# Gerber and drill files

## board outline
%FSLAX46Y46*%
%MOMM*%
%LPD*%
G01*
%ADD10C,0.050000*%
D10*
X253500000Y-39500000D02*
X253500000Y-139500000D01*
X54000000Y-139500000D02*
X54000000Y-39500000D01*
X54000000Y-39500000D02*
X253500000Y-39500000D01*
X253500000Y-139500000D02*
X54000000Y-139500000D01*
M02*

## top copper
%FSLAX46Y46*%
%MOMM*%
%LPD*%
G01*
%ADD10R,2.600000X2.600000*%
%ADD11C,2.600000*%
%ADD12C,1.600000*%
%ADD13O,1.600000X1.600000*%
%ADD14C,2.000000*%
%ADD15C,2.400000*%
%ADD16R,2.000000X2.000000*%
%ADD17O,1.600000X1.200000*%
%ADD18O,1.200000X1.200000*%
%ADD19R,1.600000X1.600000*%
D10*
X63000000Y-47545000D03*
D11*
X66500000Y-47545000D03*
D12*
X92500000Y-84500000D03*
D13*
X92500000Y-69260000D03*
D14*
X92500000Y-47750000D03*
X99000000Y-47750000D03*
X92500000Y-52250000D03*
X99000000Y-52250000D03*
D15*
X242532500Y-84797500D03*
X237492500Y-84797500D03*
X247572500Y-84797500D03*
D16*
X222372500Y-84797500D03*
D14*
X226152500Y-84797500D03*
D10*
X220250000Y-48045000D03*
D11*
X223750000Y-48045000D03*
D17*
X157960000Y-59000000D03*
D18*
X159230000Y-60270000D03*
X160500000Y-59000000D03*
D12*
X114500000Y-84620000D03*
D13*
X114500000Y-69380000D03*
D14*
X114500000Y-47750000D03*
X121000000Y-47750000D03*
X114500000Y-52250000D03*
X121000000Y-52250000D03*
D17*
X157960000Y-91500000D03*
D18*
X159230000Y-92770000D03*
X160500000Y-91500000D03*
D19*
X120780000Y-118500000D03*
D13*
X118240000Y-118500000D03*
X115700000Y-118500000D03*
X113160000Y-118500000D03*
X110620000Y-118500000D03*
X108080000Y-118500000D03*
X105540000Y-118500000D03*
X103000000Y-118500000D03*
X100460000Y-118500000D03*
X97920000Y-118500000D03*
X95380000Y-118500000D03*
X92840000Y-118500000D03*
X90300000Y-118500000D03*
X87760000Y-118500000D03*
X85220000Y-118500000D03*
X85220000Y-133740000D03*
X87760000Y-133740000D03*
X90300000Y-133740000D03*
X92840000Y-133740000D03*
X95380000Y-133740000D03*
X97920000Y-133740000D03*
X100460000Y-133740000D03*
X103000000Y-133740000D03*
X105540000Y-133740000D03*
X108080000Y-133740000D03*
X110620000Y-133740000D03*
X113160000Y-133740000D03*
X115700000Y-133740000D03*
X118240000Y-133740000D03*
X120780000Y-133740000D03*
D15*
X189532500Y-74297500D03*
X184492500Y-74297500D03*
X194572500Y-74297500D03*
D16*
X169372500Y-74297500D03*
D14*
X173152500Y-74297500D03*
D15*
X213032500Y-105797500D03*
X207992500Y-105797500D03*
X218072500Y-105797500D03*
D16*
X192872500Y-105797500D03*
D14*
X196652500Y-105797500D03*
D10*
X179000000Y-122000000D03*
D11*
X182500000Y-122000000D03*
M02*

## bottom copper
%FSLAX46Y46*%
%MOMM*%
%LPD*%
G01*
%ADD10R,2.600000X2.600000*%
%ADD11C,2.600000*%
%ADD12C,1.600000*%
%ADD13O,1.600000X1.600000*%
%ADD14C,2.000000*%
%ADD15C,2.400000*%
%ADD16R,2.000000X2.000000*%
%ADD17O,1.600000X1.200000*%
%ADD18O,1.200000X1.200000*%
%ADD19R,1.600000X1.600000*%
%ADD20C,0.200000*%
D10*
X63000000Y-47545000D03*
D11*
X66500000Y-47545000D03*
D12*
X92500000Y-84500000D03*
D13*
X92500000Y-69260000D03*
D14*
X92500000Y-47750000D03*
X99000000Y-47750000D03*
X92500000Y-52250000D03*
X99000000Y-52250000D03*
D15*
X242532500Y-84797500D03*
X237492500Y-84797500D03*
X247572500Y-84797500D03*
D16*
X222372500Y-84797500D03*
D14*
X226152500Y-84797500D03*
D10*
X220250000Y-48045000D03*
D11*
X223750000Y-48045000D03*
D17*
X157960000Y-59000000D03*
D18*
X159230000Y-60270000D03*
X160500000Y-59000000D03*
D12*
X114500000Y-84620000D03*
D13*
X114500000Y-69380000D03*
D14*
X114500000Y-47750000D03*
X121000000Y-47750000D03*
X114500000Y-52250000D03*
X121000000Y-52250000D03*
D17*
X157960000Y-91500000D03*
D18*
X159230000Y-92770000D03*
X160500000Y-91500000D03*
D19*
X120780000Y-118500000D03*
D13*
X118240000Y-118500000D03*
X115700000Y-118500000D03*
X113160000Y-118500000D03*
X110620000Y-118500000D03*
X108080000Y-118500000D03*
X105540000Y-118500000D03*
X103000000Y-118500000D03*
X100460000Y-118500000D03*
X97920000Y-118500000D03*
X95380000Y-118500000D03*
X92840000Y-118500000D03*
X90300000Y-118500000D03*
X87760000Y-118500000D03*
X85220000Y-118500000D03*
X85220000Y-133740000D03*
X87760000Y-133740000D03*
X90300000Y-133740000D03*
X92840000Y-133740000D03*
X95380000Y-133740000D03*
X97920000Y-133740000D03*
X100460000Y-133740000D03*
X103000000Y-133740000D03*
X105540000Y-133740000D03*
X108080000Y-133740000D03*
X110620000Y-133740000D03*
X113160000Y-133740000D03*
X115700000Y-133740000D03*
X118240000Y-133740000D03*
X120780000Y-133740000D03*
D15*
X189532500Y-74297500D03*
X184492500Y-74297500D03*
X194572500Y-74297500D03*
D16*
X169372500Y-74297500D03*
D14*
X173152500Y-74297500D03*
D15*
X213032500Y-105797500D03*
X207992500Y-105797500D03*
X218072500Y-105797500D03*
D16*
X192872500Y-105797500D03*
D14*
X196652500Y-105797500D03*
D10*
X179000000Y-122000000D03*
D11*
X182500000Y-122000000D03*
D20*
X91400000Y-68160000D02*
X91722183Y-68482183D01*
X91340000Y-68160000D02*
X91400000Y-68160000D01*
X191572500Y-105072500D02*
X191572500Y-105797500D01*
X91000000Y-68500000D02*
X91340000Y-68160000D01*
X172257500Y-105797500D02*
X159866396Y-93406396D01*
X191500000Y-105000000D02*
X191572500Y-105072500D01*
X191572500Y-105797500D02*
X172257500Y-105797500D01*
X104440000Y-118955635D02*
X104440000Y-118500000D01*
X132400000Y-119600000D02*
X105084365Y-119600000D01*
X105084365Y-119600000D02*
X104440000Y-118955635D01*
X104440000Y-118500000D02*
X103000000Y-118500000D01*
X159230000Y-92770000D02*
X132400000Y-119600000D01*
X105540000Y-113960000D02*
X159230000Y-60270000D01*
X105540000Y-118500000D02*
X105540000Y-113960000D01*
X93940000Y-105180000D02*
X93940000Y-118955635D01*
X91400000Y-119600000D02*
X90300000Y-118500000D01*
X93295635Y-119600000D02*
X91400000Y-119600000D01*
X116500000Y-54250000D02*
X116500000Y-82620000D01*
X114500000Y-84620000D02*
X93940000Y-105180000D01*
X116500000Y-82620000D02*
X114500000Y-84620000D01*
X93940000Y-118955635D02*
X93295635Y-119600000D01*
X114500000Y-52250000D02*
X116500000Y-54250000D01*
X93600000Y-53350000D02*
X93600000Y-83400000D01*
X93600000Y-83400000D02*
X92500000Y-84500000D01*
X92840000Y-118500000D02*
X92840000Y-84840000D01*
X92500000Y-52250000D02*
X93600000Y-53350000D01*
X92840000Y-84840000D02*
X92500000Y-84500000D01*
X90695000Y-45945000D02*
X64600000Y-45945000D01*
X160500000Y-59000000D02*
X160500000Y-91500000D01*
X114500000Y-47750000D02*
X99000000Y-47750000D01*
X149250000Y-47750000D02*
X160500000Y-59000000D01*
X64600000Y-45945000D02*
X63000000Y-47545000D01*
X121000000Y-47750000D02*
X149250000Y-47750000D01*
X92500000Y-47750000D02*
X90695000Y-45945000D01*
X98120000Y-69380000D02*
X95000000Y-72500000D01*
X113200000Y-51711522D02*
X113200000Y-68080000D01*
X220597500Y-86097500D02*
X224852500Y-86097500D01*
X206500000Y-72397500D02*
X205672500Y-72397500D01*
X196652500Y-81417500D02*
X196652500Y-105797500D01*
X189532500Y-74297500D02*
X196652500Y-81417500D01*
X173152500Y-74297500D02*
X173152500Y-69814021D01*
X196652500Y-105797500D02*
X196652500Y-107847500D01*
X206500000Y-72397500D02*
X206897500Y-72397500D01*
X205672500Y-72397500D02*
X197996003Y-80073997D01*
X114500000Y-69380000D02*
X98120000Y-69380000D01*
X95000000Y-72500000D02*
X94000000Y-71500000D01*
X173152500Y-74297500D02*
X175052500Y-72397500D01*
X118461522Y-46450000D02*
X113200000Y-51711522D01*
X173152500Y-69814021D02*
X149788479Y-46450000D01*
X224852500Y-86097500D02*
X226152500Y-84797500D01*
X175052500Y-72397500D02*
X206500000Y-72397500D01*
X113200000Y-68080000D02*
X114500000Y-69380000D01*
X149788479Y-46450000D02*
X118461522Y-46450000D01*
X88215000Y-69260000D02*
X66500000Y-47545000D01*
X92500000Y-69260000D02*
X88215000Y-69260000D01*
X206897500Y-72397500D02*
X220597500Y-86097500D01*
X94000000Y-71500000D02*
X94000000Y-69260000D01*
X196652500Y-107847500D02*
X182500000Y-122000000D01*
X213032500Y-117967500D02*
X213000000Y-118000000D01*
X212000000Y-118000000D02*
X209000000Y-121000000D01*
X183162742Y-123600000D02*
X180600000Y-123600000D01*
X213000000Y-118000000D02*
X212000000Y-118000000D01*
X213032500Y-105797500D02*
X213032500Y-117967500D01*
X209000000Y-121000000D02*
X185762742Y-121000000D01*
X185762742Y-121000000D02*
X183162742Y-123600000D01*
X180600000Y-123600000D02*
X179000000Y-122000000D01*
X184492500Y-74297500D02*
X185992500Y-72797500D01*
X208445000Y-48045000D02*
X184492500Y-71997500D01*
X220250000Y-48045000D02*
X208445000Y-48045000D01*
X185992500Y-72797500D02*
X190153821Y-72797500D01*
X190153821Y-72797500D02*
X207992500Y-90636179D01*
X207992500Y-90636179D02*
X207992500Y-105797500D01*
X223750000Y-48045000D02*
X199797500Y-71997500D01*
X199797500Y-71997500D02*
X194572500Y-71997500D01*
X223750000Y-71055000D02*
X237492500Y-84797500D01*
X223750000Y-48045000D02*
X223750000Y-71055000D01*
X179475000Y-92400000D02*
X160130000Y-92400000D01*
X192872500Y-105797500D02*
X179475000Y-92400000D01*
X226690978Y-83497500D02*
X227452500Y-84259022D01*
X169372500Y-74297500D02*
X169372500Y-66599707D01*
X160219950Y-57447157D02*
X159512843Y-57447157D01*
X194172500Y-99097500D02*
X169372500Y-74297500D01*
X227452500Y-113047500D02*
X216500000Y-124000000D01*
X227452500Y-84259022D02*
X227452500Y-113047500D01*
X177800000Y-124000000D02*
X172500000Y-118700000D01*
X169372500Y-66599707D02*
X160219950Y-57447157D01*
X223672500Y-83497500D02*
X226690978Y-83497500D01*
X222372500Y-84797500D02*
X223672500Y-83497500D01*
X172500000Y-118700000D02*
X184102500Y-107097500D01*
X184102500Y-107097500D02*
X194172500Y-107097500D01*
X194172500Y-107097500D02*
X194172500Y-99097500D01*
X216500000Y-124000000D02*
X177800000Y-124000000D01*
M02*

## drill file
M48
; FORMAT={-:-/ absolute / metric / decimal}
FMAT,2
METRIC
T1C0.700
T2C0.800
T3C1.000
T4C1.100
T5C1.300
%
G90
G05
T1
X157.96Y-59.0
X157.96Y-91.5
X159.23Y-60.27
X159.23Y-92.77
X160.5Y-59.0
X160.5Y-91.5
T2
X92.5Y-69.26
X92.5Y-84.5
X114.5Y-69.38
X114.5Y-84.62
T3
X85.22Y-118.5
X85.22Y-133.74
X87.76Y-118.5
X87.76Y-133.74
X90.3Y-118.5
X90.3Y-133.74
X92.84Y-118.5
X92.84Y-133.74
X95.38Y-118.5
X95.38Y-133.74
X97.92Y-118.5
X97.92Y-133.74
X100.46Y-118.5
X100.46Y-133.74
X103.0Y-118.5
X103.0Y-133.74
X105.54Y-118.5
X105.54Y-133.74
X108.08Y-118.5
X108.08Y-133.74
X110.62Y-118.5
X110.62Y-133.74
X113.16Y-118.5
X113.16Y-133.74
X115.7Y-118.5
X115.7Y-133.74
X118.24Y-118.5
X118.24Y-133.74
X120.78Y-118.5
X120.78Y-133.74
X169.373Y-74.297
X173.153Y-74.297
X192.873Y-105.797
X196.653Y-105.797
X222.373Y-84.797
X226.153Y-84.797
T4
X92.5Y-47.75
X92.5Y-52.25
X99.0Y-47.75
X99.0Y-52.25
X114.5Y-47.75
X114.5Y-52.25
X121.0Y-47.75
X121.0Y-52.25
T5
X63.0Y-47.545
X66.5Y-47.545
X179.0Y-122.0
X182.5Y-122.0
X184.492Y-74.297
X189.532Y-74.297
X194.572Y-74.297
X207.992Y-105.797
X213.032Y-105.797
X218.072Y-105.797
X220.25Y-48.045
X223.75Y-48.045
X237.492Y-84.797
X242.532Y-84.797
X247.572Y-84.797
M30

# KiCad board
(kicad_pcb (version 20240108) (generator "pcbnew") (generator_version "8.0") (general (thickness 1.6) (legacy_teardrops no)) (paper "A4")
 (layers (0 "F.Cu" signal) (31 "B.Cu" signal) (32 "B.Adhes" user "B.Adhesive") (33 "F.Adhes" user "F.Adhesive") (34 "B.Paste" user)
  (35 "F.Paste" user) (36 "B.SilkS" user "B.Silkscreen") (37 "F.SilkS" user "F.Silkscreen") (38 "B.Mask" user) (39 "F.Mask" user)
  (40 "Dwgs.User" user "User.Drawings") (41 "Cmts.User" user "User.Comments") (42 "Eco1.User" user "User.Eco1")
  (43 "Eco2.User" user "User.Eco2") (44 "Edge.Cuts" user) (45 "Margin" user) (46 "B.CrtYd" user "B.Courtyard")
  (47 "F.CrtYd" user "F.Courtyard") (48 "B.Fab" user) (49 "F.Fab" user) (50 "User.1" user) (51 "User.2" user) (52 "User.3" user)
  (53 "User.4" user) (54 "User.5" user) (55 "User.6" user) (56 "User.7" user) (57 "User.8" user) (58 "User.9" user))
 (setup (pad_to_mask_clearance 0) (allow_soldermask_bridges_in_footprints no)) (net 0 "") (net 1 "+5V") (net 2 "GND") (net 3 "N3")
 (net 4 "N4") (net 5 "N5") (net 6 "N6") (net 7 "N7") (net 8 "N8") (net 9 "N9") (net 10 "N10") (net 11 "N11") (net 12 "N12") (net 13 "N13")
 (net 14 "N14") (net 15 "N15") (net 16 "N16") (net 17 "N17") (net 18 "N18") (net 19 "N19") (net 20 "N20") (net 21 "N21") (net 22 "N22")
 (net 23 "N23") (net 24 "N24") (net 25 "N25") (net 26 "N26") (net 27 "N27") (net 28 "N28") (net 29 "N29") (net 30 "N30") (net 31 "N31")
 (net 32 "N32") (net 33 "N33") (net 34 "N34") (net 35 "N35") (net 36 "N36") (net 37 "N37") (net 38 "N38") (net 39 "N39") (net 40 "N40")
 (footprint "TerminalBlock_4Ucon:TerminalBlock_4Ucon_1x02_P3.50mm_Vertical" (layer "F.Cu") (at 63 47.545)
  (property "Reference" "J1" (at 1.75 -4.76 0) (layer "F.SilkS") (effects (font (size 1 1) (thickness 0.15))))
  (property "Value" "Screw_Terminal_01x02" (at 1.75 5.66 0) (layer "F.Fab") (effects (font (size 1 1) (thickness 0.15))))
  (pad "1" thru_hole rect (at 0 0) (size 2.6 2.6) (drill 1.3) (layers "*.Cu" "*.Mask") (remove_unused_layers no) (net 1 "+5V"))
  (pad "2" thru_hole circle (at 3.5 0) (size 2.6 2.6) (drill 1.3) (layers "*.Cu" "*.Mask") (remove_unused_layers no) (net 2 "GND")))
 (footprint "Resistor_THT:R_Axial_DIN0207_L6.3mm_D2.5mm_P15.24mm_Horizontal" (layer "F.Cu") (at 92.5 84.5 90)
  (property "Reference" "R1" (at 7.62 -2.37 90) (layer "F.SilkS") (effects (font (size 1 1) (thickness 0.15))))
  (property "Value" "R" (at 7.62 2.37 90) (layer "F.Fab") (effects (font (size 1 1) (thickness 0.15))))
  (pad "1" thru_hole circle (at 0 0 90) (size 1.6 1.6) (drill 0.8) (layers "*.Cu" "*.Mask") (remove_unused_layers no) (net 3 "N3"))
  (pad "2" thru_hole oval (at 15.24 0 90) (size 1.6 1.6) (drill 0.8) (layers "*.Cu" "*.Mask") (remove_unused_layers no) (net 2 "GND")))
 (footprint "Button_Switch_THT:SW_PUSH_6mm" (layer "F.Cu") (at 92.5 47.75)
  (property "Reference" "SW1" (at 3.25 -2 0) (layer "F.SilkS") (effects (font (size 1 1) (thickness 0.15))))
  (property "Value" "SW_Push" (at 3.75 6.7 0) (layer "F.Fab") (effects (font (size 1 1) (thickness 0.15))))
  (pad "1" thru_hole circle (at 0 0 90) (size 2 2) (drill 1.1) (layers "*.Cu" "*.Mask") (remove_unused_layers no) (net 1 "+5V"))
  (pad "1" thru_hole circle (at 6.5 0 90) (size 2 2) (drill 1.1) (layers "*.Cu" "*.Mask") (remove_unused_layers no) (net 1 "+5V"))
  (pad "2" thru_hole circle (at 0 4.5 90) (size 2 2) (drill 1.1) (layers "*.Cu" "*.Mask") (remove_unused_layers no) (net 3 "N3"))
  (pad "2" thru_hole circle (at 6.5 4.5 90) (size 2 2) (drill 1.1) (layers "*.Cu" "*.Mask") (remove_unused_layers no) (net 3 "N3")))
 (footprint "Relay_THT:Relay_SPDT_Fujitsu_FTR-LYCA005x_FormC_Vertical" (layer "F.Cu") (at 222.3725 84.7975)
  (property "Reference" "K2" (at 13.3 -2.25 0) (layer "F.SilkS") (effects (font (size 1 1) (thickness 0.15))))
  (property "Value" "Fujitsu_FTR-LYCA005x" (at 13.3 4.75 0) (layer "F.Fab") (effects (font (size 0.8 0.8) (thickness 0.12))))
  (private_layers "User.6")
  (pad "11" thru_hole circle (at 20.16 0) (size 2.4 2.4) (drill 1.3) (layers "*.Cu" "*.Mask") (remove_unused_layers no) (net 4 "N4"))
  (pad "12" thru_hole circle (at 15.12 0) (size 2.4 2.4) (drill 1.3) (layers "*.Cu" "*.Mask") (remove_unused_layers no) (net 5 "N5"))
  (pad "14" thru_hole circle (at 25.2 0) (size 2.4 2.4) (drill 1.3) (layers "*.Cu" "*.Mask") (remove_unused_layers no) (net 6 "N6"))
  (pad "A1" thru_hole rect (at 0 0) (size 2 2) (drill 1) (layers "*.Cu" "*.Mask") (remove_unused_layers no) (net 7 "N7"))
  (pad "A2" thru_hole circle (at 3.78 0) (size 2 2) (drill 1) (layers "*.Cu" "*.Mask") (remove_unused_layers no) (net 2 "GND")))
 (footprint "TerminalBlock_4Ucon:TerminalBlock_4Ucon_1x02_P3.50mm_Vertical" (layer "F.Cu") (at 220.25 48.045)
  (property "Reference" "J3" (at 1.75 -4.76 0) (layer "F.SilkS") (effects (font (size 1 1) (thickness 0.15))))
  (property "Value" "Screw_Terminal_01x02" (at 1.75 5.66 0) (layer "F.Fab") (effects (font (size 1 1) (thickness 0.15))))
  (pad "1" thru_hole rect (at 0 0) (size 2.6 2.6) (drill 1.3) (layers "*.Cu" "*.Mask") (remove_unused_layers no) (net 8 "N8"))
  (pad "2" thru_hole circle (at 3.5 0) (size 2.6 2.6) (drill 1.3) (layers "*.Cu" "*.Mask") (remove_unused_layers no) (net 5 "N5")))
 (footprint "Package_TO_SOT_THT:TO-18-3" (layer "F.Cu") (at 157.96 59)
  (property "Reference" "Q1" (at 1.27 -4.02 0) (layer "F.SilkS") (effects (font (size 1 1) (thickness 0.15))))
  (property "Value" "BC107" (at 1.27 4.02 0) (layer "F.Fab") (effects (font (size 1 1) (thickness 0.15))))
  (pad "1" thru_hole oval (at 0 0) (size 1.6 1.2) (drill 0.7) (layers "*.Cu" "*.Mask") (remove_unused_layers no) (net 7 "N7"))
  (pad "2" thru_hole oval (at 1.27 1.27) (size 1.2 1.2) (drill 0.7) (layers "*.Cu" "*.Mask") (remove_unused_layers no) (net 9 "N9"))
  (pad "3" thru_hole oval (at 2.54 0) (size 1.2 1.2) (drill 0.7) (layers "*.Cu" "*.Mask") (remove_unused_layers no) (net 1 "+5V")))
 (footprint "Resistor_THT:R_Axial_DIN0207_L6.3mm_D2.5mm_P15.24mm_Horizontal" (layer "F.Cu") (at 114.5 84.62 90)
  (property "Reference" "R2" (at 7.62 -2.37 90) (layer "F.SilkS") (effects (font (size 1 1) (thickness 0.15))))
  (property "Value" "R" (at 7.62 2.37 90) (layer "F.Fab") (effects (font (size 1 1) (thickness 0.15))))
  (pad "1" thru_hole circle (at 0 0 90) (size 1.6 1.6) (drill 0.8) (layers "*.Cu" "*.Mask") (remove_unused_layers no) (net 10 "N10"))
  (pad "2" thru_hole oval (at 15.24 0 90) (size 1.6 1.6) (drill 0.8) (layers "*.Cu" "*.Mask") (remove_unused_layers no) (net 2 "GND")))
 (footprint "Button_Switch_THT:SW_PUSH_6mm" (layer "F.Cu") (at 114.5 47.75)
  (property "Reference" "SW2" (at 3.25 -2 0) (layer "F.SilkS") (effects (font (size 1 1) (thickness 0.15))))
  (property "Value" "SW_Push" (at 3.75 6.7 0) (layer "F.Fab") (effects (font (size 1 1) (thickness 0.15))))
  (pad "1" thru_hole circle (at 0 0 90) (size 2 2) (drill 1.1) (layers "*.Cu" "*.Mask") (remove_unused_layers no) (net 1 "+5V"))
  (pad "1" thru_hole circle (at 6.5 0 90) (size 2 2) (drill 1.1) (layers "*.Cu" "*.Mask") (remove_unused_layers no) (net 1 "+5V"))
  (pad "2" thru_hole circle (at 0 4.5 90) (size 2 2) (drill 1.1) (layers "*.Cu" "*.Mask") (remove_unused_layers no) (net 10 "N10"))
  (pad "2" thru_hole circle (at 6.5 4.5 90) (size 2 2) (drill 1.1) (layers "*.Cu" "*.Mask") (remove_unused_layers no) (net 10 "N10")))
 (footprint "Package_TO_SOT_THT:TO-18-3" (layer "F.Cu") (at 157.96 91.5)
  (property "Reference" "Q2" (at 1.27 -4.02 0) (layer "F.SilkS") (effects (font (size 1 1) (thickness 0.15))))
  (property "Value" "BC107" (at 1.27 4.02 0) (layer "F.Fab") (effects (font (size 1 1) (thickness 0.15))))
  (pad "1" thru_hole oval (at 0 0) (size 1.6 1.2) (drill 0.7) (layers "*.Cu" "*.Mask") (remove_unused_layers no) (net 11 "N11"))
  (pad "2" thru_hole oval (at 1.27 1.27) (size 1.2 1.2) (drill 0.7) (layers "*.Cu" "*.Mask") (remove_unused_layers no) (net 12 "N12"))
  (pad "3" thru_hole oval (at 2.54 0) (size 1.2 1.2) (drill 0.7) (layers "*.Cu" "*.Mask") (remove_unused_layers no) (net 1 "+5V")))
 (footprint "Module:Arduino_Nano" (layer "F.Cu") (at 120.78 118.5 -90)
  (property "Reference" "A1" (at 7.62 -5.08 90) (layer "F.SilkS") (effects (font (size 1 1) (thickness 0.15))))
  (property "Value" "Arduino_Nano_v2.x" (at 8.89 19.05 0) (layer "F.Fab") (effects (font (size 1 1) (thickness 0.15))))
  (pad "1" thru_hole rect (at 0 0 270) (size 1.6 1.6) (drill 1) (layers "*.Cu" "*.Mask") (remove_unused_layers no) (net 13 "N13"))
  (pad "2" thru_hole oval (at 0 2.54 270) (size 1.6 1.6) (drill 1) (layers "*.Cu" "*.Mask") (remove_unused_layers no) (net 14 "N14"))
  (pad "3" thru_hole oval (at 0 5.08 270) (size 1.6 1.6) (drill 1) (layers "*.Cu" "*.Mask") (remove_unused_layers no) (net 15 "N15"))
  (pad "4" thru_hole oval (at 0 7.62 270) (size 1.6 1.6) (drill 1) (layers "*.Cu" "*.Mask") (remove_unused_layers no) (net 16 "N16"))
  (pad "5" thru_hole oval (at 0 10.16 270) (size 1.6 1.6) (drill 1) (layers "*.Cu" "*.Mask") (remove_unused_layers no) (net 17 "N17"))
  (pad "6" thru_hole oval (at 0 12.7 270) (size 1.6 1.6) (drill 1) (layers "*.Cu" "*.Mask") (remove_unused_layers no) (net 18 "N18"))
  (pad "7" thru_hole oval (at 0 15.24 270) (size 1.6 1.6) (drill 1) (layers "*.Cu" "*.Mask") (remove_unused_layers no) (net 9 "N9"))
  (pad "8" thru_hole oval (at 0 17.78 270) (size 1.6 1.6) (drill 1) (layers "*.Cu" "*.Mask") (remove_unused_layers no) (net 12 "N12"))
  (pad "9" thru_hole oval (at 0 20.32 270) (size 1.6 1.6) (drill 1) (layers "*.Cu" "*.Mask") (remove_unused_layers no) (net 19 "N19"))
  (pad "10" thru_hole oval (at 0 22.86 270) (size 1.6 1.6) (drill 1) (layers "*.Cu" "*.Mask") (remove_unused_layers no) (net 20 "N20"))
  (pad "11" thru_hole oval (at 0 25.4 270) (size 1.6 1.6) (drill 1) (layers "*.Cu" "*.Mask") (remove_unused_layers no) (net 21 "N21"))
  (pad "12" thru_hole oval (at 0 27.94 270) (size 1.6 1.6) (drill 1) (layers "*.Cu" "*.Mask") (remove_unused_layers no) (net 3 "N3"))
  (pad "13" thru_hole oval (at 0 30.48 270) (size 1.6 1.6) (drill 1) (layers "*.Cu" "*.Mask") (remove_unused_layers no) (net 10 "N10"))
  (pad "14" thru_hole oval (at 0 33.02 270) (size 1.6 1.6) (drill 1) (layers "*.Cu" "*.Mask") (remove_unused_layers no) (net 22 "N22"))
  (pad "15" thru_hole oval (at 0 35.56 270) (size 1.6 1.6) (drill 1) (layers "*.Cu" "*.Mask") (remove_unused_layers no) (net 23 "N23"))
  (pad "16" thru_hole oval (at 15.24 35.56 270) (size 1.6 1.6) (drill 1) (layers "*.Cu" "*.Mask") (remove_unused_layers no) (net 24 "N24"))
  (pad "17" thru_hole oval (at 15.24 33.02 270) (size 1.6 1.6) (drill 1) (layers "*.Cu" "*.Mask") (remove_unused_layers no) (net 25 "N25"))
  (pad "18" thru_hole oval (at 15.24 30.48 270) (size 1.6 1.6) (drill 1) (layers "*.Cu" "*.Mask") (remove_unused_layers no) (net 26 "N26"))
  (pad "19" thru_hole oval (at 15.24 27.94 270) (size 1.6 1.6) (drill 1) (layers "*.Cu" "*.Mask") (remove_unused_layers no) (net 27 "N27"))
  (pad "20" thru_hole oval (at 15.24 25.4 270) (size 1.6 1.6) (drill 1) (layers "*.Cu" "*.Mask") (remove_unused_layers no) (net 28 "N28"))
  (pad "21" thru_hole oval (at 15.24 22.86 270) (size 1.6 1.6) (drill 1) (layers "*.Cu" "*.Mask") (remove_unused_layers no) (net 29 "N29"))
  (pad "22" thru_hole oval (at 15.24 20.32 270) (size 1.6 1.6) (drill 1) (layers "*.Cu" "*.Mask") (remove_unused_layers no) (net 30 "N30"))
  (pad "23" thru_hole oval (at 15.24 17.78 270) (size 1.6 1.6) (drill 1) (layers "*.Cu" "*.Mask") (remove_unused_layers no) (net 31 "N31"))
  (pad "24" thru_hole oval (at 15.24 15.24 270) (size 1.6 1.6) (drill 1) (layers "*.Cu" "*.Mask") (remove_unused_layers no) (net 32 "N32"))
  (pad "25" thru_hole oval (at 15.24 12.7 270) (size 1.6 1.6) (drill 1) (layers "*.Cu" "*.Mask") (remove_unused_layers no) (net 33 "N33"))
  (pad "26" thru_hole oval (at 15.24 10.16 270) (size 1.6 1.6) (drill 1) (layers "*.Cu" "*.Mask") (remove_unused_layers no) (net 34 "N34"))
  (pad "27" thru_hole oval (at 15.24 7.62 270) (size 1.6 1.6) (drill 1) (layers "*.Cu" "*.Mask") (remove_unused_layers no) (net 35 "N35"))
  (pad "28" thru_hole oval (at 15.24 5.08 270) (size 1.6 1.6) (drill 1) (layers "*.Cu" "*.Mask") (remove_unused_layers no) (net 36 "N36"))
  (pad "29" thru_hole oval (at 15.24 2.54 270) (size 1.6 1.6) (drill 1) (layers "*.Cu" "*.Mask") (remove_unused_layers no) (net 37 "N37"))
  (pad "30" thru_hole oval (at 15.24 0 270) (size 1.6 1.6) (drill 1) (layers "*.Cu" "*.Mask") (remove_unused_layers no) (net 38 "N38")))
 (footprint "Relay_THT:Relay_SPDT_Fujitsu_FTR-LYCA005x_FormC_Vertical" (layer "F.Cu") (at 169.3725 74.2975)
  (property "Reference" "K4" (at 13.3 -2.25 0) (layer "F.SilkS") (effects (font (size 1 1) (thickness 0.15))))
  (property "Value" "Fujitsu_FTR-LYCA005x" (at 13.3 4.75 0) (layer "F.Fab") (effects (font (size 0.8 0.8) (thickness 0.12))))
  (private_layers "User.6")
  (pad "11" thru_hole circle (at 20.16 0) (size 2.4 2.4) (drill 1.3) (layers "*.Cu" "*.Mask") (remove_unused_layers no) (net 2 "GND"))
  (pad "12" thru_hole circle (at 15.12 0) (size 2.4 2.4) (drill 1.3) (layers "*.Cu" "*.Mask") (remove_unused_layers no) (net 8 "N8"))
  (pad "14" thru_hole circle (at 25.2 0) (size 2.4 2.4) (drill 1.3) (layers "*.Cu" "*.Mask") (remove_unused_layers no) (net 5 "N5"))
  (pad "A1" thru_hole rect (at 0 0) (size 2 2) (drill 1) (layers "*.Cu" "*.Mask") (remove_unused_layers no) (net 7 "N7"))
  (pad "A2" thru_hole circle (at 3.78 0) (size 2 2) (drill 1) (layers "*.Cu" "*.Mask") (remove_unused_layers no) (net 2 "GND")))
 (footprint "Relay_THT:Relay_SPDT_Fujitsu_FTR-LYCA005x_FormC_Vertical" (layer "F.Cu") (at 192.8725 105.7975)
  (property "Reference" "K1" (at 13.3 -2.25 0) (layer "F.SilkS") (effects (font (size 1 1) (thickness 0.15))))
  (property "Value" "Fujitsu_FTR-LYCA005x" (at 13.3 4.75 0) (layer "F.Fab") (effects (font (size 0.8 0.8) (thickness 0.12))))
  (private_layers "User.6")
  (pad "11" thru_hole circle (at 20.16 0) (size 2.4 2.4) (drill 1.3) (layers "*.Cu" "*.Mask") (remove_unused_layers no) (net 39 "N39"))
  (pad "12" thru_hole circle (at 15.12 0) (size 2.4 2.4) (drill 1.3) (layers "*.Cu" "*.Mask") (remove_unused_layers no) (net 8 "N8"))
  (pad "14" thru_hole circle (at 25.2 0) (size 2.4 2.4) (drill 1.3) (layers "*.Cu" "*.Mask") (remove_unused_layers no) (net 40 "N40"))
  (pad "A1" thru_hole rect (at 0 0) (size 2 2) (drill 1) (layers "*.Cu" "*.Mask") (remove_unused_layers no) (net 11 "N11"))
  (pad "A2" thru_hole circle (at 3.78 0) (size 2 2) (drill 1) (layers "*.Cu" "*.Mask") (remove_unused_layers no) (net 2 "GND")))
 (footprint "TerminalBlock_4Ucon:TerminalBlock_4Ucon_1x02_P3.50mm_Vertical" (layer "F.Cu") (at 179 122)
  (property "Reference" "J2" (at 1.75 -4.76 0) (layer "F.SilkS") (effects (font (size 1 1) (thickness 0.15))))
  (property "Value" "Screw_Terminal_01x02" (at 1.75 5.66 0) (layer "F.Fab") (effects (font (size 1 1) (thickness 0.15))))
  (pad "1" thru_hole rect (at 0 0) (size 2.6 2.6) (drill 1.3) (layers "*.Cu" "*.Mask") (remove_unused_layers no) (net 39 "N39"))
  (pad "2" thru_hole circle (at 3.5 0) (size 2.6 2.6) (drill 1.3) (layers "*.Cu" "*.Mask") (remove_unused_layers no) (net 2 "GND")))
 (gr_line (start 253.5 39.5) (end 253.5 139.5) (stroke (width 0.05) (type default)) (layer "Edge.Cuts"))
 (gr_line (start 54 139.5) (end 54 39.5) (stroke (width 0.05) (type default)) (layer "Edge.Cuts"))
 (gr_line (start 54 39.5) (end 253.5 39.5) (stroke (width 0.05) (type default)) (layer "Edge.Cuts"))
 (gr_line (start 253.5 139.5) (end 54 139.5) (stroke (width 0.05) (type default)) (layer "Edge.Cuts"))
 (segment (start 91.4 68.16) (end 91.722183 68.482183) (width 0.2) (layer "B.Cu") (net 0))
 (segment (start 91.34 68.16) (end 91.4 68.16) (width 0.2) (layer "B.Cu") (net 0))
 (segment (start 191.5725 105.0725) (end 191.5725 105.7975) (width 0.2) (layer "B.Cu") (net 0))
 (segment (start 91 68.5) (end 91.34 68.16) (width 0.2) (layer "B.Cu") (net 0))
 (segment (start 172.2575 105.7975) (end 159.866396 93.406396) (width 0.2) (layer "B.Cu") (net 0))
 (segment (start 191.5 105) (end 191.5725 105.0725) (width 0.2) (layer "B.Cu") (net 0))
 (segment (start 191.5725 105.7975) (end 172.2575 105.7975) (width 0.2) (layer "B.Cu") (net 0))
 (segment (start 104.44 118.955635) (end 104.44 118.5) (width 0.2) (layer "B.Cu") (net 12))
 (segment (start 132.4 119.6) (end 105.084365 119.6) (width 0.2) (layer "B.Cu") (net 12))
 (segment (start 105.084365 119.6) (end 104.44 118.955635) (width 0.2) (layer "B.Cu") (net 12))
 (segment (start 104.44 118.5) (end 103 118.5) (width 0.2) (layer "B.Cu") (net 12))
 (segment (start 159.23 92.77) (end 132.4 119.6) (width 0.2) (layer "B.Cu") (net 12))
 (segment (start 105.54 113.96) (end 159.23 60.27) (width 0.2) (layer "B.Cu") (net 9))
 (segment (start 105.54 118.5) (end 105.54 113.96) (width 0.2) (layer "B.Cu") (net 9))
 (segment (start 93.94 105.18) (end 93.94 118.955635) (width 0.2) (layer "B.Cu") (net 10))
 (segment (start 91.4 119.6) (end 90.3 118.5) (width 0.2) (layer "B.Cu") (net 10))
 (segment (start 93.295635 119.6) (end 91.4 119.6) (width 0.2) (layer "B.Cu") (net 10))
 (segment (start 116.5 54.25) (end 116.5 82.62) (width 0.2) (layer "B.Cu") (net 10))
 (segment (start 114.5 84.62) (end 93.94 105.18) (width 0.2) (layer "B.Cu") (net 10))
 (segment (start 116.5 82.62) (end 114.5 84.62) (width 0.2) (layer "B.Cu") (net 10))
 (segment (start 93.94 118.955635) (end 93.295635 119.6) (width 0.2) (layer "B.Cu") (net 10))
 (segment (start 114.5 52.25) (end 116.5 54.25) (width 0.2) (layer "B.Cu") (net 10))
 (segment (start 93.6 53.35) (end 93.6 83.4) (width 0.2) (layer "B.Cu") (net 3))
 (segment (start 93.6 83.4) (end 92.5 84.5) (width 0.2) (layer "B.Cu") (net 3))
 (segment (start 92.84 118.5) (end 92.84 84.84) (width 0.2) (layer "B.Cu") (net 3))
 (segment (start 92.5 52.25) (end 93.6 53.35) (width 0.2) (layer "B.Cu") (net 3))
 (segment (start 92.84 84.84) (end 92.5 84.5) (width 0.2) (layer "B.Cu") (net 3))
 (segment (start 90.695 45.945) (end 64.6 45.945) (width 0.2) (layer "B.Cu") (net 1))
 (segment (start 160.5 59) (end 160.5 91.5) (width 0.2) (layer "B.Cu") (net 1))
 (segment (start 114.5 47.75) (end 99 47.75) (width 0.2) (layer "B.Cu") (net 1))
 (segment (start 149.25 47.75) (end 160.5 59) (width 0.2) (layer "B.Cu") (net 1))
 (segment (start 64.6 45.945) (end 63 47.545) (width 0.2) (layer "B.Cu") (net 1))
 (segment (start 121 47.75) (end 149.25 47.75) (width 0.2) (layer "B.Cu") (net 1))
 (segment (start 92.5 47.75) (end 90.695 45.945) (width 0.2) (layer "B.Cu") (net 1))
 (segment (start 98.12 69.38) (end 95 72.5) (width 0.2) (layer "B.Cu") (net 2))
 (segment (start 113.2 51.711522) (end 113.2 68.08) (width 0.2) (layer "B.Cu") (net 2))
 (segment (start 220.5975 86.0975) (end 224.8525 86.0975) (width 0.2) (layer "B.Cu") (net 2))
 (segment (start 206.5 72.3975) (end 205.6725 72.3975) (width 0.2) (layer "B.Cu") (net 2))
 (segment (start 196.6525 81.4175) (end 196.6525 105.7975) (width 0.2) (layer "B.Cu") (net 2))
 (segment (start 189.5325 74.2975) (end 196.6525 81.4175) (width 0.2) (layer "B.Cu") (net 2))
 (segment (start 173.1525 74.2975) (end 173.1525 69.814021) (width 0.2) (layer "B.Cu") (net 2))
 (segment (start 196.6525 105.7975) (end 196.6525 107.8475) (width 0.2) (layer "B.Cu") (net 2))
 (segment (start 206.5 72.3975) (end 206.8975 72.3975) (width 0.2) (layer "B.Cu") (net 2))
 (segment (start 205.6725 72.3975) (end 197.996003 80.073997) (width 0.2) (layer "B.Cu") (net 2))
 (segment (start 114.5 69.38) (end 98.12 69.38) (width 0.2) (layer "B.Cu") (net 2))
 (segment (start 95 72.5) (end 94 71.5) (width 0.2) (layer "B.Cu") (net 2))
 (segment (start 173.1525 74.2975) (end 175.0525 72.3975) (width 0.2) (layer "B.Cu") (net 2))
 (segment (start 118.461522 46.45) (end 113.2 51.711522) (width 0.2) (layer "B.Cu") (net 2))
 (segment (start 173.1525 69.814021) (end 149.788479 46.45) (width 0.2) (layer "B.Cu") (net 2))
 (segment (start 224.8525 86.0975) (end 226.1525 84.7975) (width 0.2) (layer "B.Cu") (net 2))
 (segment (start 175.0525 72.3975) (end 206.5 72.3975) (width 0.2) (layer "B.Cu") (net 2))
 (segment (start 113.2 68.08) (end 114.5 69.38) (width 0.2) (layer "B.Cu") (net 2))
 (segment (start 149.788479 46.45) (end 118.461522 46.45) (width 0.2) (layer "B.Cu") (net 2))
 (segment (start 88.215 69.26) (end 66.5 47.545) (width 0.2) (layer "B.Cu") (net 2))
 (segment (start 92.5 69.26) (end 88.215 69.26) (width 0.2) (layer "B.Cu") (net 2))
 (segment (start 206.8975 72.3975) (end 220.5975 86.0975) (width 0.2) (layer "B.Cu") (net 2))
 (segment (start 94 71.5) (end 94 69.26) (width 0.2) (layer "B.Cu") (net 2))
 (segment (start 196.6525 107.8475) (end 182.5 122) (width 0.2) (layer "B.Cu") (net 2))
 (segment (start 213.0325 117.9675) (end 213 118) (width 0.2) (layer "B.Cu") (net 39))
 (segment (start 212 118) (end 209 121) (width 0.2) (layer "B.Cu") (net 39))
 (segment (start 183.162742 123.6) (end 180.6 123.6) (width 0.2) (layer "B.Cu") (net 39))
 (segment (start 213 118) (end 212 118) (width 0.2) (layer "B.Cu") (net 39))
 (segment (start 213.0325 105.7975) (end 213.0325 117.9675) (width 0.2) (layer "B.Cu") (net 39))
 (segment (start 209 121) (end 185.762742 121) (width 0.2) (layer "B.Cu") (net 39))
 (segment (start 185.762742 121) (end 183.162742 123.6) (width 0.2) (layer "B.Cu") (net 39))
 (segment (start 180.6 123.6) (end 179 122) (width 0.2) (layer "B.Cu") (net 39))
 (segment (start 184.4925 74.2975) (end 185.9925 72.7975) (width 0.2) (layer "B.Cu") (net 8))
 (segment (start 208.445 48.045) (end 184.4925 71.9975) (width 0.2) (layer "B.Cu") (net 8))
 (segment (start 220.25 48.045) (end 208.445 48.045) (width 0.2) (layer "B.Cu") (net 8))
 (segment (start 185.9925 72.7975) (end 190.153821 72.7975) (width 0.2) (layer "B.Cu") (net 8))
 (segment (start 190.153821 72.7975) (end 207.9925 90.636179) (width 0.2) (layer "B.Cu") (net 8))
 (segment (start 207.9925 90.636179) (end 207.9925 105.7975) (width 0.2) (layer "B.Cu") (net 8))
 (segment (start 223.75 48.045) (end 199.7975 71.9975) (width 0.2) (layer "B.Cu") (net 5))
 (segment (start 199.7975 71.9975) (end 194.5725 71.9975) (width 0.2) (layer "B.Cu") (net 5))
 (segment (start 223.75 71.055) (end 237.4925 84.7975) (width 0.2) (layer "B.Cu") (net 5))
 (segment (start 223.75 48.045) (end 223.75 71.055) (width 0.2) (layer "B.Cu") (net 5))
 (segment (start 179.475 92.4) (end 160.13 92.4) (width 0.2) (layer "B.Cu") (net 11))
 (segment (start 192.8725 105.7975) (end 179.475 92.4) (width 0.2) (layer "B.Cu") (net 11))
 (segment (start 226.690978 83.4975) (end 227.4525 84.259022) (width 0.2) (layer "B.Cu") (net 7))
 (segment (start 169.3725 74.2975) (end 169.3725 66.599707) (width 0.2) (layer "B.Cu") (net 7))
 (segment (start 160.21995 57.447157) (end 159.512843 57.447157) (width 0.2) (layer "B.Cu") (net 7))
 (segment (start 194.1725 99.0975) (end 169.3725 74.2975) (width 0.2) (layer "B.Cu") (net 7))
 (segment (start 227.4525 113.0475) (end 216.5 124) (width 0.2) (layer "B.Cu") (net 7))
 (segment (start 227.4525 84.259022) (end 227.4525 113.0475) (width 0.2) (layer "B.Cu") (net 7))
 (segment (start 177.8 124) (end 172.5 118.7) (width 0.2) (layer "B.Cu") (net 7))
 (segment (start 169.3725 66.599707) (end 160.21995 57.447157) (width 0.2) (layer "B.Cu") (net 7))
 (segment (start 223.6725 83.4975) (end 226.690978 83.4975) (width 0.2) (layer "B.Cu") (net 7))
 (segment (start 222.3725 84.7975) (end 223.6725 83.4975) (width 0.2) (layer "B.Cu") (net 7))
 (segment (start 172.5 118.7) (end 184.1025 107.0975) (width 0.2) (layer "B.Cu") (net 7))
 (segment (start 184.1025 107.0975) (end 194.1725 107.0975) (width 0.2) (layer "B.Cu") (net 7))
 (segment (start 194.1725 107.0975) (end 194.1725 99.0975) (width 0.2) (layer "B.Cu") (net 7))
 (segment (start 216.5 124) (end 177.8 124) (width 0.2) (layer "B.Cu") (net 7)))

